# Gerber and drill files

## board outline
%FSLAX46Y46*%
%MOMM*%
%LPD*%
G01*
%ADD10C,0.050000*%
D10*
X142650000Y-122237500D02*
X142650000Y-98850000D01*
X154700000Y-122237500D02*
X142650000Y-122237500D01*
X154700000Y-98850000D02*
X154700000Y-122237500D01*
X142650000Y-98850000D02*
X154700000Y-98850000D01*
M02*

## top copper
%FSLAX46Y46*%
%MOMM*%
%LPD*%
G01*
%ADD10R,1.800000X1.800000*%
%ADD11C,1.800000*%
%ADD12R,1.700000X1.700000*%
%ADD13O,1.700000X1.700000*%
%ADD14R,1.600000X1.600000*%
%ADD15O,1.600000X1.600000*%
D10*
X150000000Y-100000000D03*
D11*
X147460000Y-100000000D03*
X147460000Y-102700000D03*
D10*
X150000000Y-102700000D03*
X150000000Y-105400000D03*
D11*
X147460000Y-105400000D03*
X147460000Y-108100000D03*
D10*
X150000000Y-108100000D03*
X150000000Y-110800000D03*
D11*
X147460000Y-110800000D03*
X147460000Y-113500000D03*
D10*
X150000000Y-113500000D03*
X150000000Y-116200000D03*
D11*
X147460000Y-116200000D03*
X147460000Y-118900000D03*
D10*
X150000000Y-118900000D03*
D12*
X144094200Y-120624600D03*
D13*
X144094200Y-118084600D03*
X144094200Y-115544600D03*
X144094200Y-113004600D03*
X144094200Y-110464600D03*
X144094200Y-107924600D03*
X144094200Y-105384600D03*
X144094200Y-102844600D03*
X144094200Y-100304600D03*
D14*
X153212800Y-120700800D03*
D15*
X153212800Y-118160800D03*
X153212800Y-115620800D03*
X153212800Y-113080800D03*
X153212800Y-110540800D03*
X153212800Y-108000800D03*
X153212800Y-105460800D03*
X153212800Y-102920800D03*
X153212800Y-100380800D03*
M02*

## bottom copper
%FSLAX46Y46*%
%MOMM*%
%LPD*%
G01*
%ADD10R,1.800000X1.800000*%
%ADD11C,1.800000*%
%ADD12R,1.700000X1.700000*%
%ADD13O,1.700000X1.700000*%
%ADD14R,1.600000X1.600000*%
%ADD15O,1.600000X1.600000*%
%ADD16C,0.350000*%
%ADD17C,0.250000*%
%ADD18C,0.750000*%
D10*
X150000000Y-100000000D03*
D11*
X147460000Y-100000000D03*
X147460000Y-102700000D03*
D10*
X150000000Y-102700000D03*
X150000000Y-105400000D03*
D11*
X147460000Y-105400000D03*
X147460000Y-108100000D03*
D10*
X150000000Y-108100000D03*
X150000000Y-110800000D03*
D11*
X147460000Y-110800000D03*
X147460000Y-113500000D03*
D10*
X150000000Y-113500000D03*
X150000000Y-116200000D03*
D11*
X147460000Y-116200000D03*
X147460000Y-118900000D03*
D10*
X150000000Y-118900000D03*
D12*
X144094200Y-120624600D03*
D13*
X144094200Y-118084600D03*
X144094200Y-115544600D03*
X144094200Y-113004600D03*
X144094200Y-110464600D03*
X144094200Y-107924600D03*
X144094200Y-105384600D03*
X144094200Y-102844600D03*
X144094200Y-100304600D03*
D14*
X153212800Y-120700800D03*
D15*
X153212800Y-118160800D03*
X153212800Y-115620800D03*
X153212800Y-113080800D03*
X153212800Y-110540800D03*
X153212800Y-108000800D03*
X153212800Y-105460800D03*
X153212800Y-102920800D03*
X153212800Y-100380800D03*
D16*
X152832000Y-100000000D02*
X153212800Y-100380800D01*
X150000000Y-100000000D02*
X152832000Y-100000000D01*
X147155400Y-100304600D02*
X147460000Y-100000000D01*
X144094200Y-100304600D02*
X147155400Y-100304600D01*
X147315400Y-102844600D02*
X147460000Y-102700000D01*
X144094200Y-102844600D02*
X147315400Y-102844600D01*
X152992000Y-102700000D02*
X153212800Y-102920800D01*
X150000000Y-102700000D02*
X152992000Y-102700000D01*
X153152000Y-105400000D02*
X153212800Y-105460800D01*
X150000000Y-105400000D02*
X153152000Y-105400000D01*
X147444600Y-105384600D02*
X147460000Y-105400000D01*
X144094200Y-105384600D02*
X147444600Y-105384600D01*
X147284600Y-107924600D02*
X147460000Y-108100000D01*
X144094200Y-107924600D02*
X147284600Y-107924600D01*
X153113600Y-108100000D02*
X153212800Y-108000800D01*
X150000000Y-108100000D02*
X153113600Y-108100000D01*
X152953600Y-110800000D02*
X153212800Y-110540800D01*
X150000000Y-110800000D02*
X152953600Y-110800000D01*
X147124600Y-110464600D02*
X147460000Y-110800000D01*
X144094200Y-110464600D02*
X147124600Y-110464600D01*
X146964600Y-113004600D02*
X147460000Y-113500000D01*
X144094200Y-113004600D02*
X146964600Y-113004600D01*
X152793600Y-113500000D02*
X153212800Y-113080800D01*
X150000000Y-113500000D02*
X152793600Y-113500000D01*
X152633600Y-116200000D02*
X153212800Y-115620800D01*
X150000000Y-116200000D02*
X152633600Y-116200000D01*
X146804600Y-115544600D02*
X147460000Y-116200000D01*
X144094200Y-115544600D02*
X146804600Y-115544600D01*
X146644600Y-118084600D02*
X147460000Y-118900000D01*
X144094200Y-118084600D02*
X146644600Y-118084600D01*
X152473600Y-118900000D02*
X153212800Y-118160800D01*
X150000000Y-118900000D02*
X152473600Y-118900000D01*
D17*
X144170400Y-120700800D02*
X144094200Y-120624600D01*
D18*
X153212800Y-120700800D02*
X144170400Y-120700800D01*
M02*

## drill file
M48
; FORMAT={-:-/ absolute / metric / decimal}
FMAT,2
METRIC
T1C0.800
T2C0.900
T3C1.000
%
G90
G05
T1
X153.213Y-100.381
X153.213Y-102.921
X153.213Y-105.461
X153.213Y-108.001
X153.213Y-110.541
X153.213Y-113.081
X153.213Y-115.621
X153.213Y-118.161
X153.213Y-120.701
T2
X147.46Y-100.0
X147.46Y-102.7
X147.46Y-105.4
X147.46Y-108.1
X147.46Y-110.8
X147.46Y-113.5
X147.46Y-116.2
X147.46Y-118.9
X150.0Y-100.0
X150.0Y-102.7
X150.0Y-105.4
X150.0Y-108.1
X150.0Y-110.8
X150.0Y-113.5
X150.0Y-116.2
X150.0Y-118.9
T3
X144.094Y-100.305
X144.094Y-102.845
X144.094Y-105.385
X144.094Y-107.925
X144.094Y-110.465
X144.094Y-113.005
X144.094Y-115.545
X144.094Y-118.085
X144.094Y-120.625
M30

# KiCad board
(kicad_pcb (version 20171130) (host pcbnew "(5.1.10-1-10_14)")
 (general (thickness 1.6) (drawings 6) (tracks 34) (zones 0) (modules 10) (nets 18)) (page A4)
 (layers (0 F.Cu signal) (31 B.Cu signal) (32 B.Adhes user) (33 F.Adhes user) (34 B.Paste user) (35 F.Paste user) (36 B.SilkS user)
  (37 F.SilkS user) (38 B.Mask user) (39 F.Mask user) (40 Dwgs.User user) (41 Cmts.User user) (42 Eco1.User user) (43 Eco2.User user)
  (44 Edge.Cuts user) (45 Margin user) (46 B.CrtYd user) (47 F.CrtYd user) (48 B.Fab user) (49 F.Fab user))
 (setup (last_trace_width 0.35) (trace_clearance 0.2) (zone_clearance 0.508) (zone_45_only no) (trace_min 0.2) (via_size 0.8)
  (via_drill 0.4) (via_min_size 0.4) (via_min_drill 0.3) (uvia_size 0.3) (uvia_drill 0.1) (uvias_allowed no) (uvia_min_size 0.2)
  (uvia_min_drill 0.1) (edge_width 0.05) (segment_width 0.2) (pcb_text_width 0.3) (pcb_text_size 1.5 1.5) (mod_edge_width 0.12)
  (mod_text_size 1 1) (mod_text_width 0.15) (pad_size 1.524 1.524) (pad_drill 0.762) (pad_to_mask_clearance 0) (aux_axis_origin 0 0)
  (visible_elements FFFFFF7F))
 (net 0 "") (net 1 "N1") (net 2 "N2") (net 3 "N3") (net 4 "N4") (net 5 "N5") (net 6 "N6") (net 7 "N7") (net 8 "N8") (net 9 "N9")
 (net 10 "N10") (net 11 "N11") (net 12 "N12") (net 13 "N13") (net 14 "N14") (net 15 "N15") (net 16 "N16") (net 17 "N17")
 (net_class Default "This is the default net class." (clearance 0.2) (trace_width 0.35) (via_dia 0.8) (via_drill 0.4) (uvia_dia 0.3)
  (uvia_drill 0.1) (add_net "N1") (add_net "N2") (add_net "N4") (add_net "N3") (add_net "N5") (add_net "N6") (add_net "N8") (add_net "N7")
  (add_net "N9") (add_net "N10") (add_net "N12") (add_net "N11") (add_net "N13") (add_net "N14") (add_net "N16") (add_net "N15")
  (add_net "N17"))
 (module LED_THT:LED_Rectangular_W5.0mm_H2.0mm (layer F.Cu) (at 150 100 180)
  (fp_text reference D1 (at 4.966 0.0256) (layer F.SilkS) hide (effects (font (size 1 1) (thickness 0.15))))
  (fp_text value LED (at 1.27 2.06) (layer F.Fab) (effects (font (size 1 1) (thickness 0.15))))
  (pad 1 thru_hole rect (at 0 0 180) (size 1.8 1.8) (drill 0.9) (layers *.Cu *.Mask) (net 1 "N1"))
  (pad 2 thru_hole circle (at 2.54 0 180) (size 1.8 1.8) (drill 0.9) (layers *.Cu *.Mask) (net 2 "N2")))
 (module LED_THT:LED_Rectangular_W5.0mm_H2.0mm (layer F.Cu) (at 150 102.7 180)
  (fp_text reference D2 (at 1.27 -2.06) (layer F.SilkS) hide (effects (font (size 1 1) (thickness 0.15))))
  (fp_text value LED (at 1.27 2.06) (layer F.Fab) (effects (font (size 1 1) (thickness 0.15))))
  (pad 2 thru_hole circle (at 2.54 0 180) (size 1.8 1.8) (drill 0.9) (layers *.Cu *.Mask) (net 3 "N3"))
  (pad 1 thru_hole rect (at 0 0 180) (size 1.8 1.8) (drill 0.9) (layers *.Cu *.Mask) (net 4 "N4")))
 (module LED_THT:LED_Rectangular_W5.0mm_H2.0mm (layer F.Cu) (at 150 105.4 180)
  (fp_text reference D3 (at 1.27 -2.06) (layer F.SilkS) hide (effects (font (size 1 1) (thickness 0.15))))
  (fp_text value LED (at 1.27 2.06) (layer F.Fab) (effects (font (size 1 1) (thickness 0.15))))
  (pad 1 thru_hole rect (at 0 0 180) (size 1.8 1.8) (drill 0.9) (layers *.Cu *.Mask) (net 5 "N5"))
  (pad 2 thru_hole circle (at 2.54 0 180) (size 1.8 1.8) (drill 0.9) (layers *.Cu *.Mask) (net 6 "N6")))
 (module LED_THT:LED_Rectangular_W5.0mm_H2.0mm (layer F.Cu) (at 150 108.1 180)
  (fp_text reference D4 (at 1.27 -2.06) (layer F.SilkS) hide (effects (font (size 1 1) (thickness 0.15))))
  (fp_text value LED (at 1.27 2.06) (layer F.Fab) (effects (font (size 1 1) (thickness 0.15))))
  (pad 2 thru_hole circle (at 2.54 0 180) (size 1.8 1.8) (drill 0.9) (layers *.Cu *.Mask) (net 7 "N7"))
  (pad 1 thru_hole rect (at 0 0 180) (size 1.8 1.8) (drill 0.9) (layers *.Cu *.Mask) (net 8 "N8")))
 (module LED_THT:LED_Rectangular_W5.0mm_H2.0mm (layer F.Cu) (at 150 110.8 180)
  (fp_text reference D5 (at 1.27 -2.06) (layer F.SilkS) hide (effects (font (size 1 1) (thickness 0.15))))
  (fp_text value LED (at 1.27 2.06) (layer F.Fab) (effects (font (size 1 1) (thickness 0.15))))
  (pad 1 thru_hole rect (at 0 0 180) (size 1.8 1.8) (drill 0.9) (layers *.Cu *.Mask) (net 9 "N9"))
  (pad 2 thru_hole circle (at 2.54 0 180) (size 1.8 1.8) (drill 0.9) (layers *.Cu *.Mask) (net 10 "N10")))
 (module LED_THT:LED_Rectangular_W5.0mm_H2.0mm (layer F.Cu) (at 150 113.5 180)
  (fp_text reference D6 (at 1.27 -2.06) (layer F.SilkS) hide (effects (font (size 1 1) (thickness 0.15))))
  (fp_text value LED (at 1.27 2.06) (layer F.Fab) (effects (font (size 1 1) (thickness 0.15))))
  (pad 2 thru_hole circle (at 2.54 0 180) (size 1.8 1.8) (drill 0.9) (layers *.Cu *.Mask) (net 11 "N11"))
  (pad 1 thru_hole rect (at 0 0 180) (size 1.8 1.8) (drill 0.9) (layers *.Cu *.Mask) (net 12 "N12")))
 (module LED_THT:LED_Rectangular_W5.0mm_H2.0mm (layer F.Cu) (at 150 116.2 180)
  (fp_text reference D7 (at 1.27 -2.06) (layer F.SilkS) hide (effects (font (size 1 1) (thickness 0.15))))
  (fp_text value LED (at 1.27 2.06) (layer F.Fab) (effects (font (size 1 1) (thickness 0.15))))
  (pad 1 thru_hole rect (at 0 0 180) (size 1.8 1.8) (drill 0.9) (layers *.Cu *.Mask) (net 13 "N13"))
  (pad 2 thru_hole circle (at 2.54 0 180) (size 1.8 1.8) (drill 0.9) (layers *.Cu *.Mask) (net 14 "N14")))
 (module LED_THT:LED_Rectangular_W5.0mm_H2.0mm (layer F.Cu) (at 150 118.9 180)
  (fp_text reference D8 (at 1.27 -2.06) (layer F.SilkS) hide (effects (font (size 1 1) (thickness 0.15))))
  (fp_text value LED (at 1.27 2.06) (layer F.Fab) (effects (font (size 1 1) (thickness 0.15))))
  (pad 2 thru_hole circle (at 2.54 0 180) (size 1.8 1.8) (drill 0.9) (layers *.Cu *.Mask) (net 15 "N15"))
  (pad 1 thru_hole rect (at 0 0 180) (size 1.8 1.8) (drill 0.9) (layers *.Cu *.Mask) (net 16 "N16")))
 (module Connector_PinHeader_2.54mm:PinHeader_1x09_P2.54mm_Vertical (layer F.Cu) (at 144.0942 120.6246 180)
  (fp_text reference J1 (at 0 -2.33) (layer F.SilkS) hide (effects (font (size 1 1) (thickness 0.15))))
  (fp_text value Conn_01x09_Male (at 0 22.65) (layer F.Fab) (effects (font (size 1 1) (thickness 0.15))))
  (pad 1 thru_hole rect (at 0 0 180) (size 1.7 1.7) (drill 1) (layers *.Cu *.Mask) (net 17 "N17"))
  (pad 2 thru_hole oval (at 0 2.54 180) (size 1.7 1.7) (drill 1) (layers *.Cu *.Mask) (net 15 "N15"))
  (pad 3 thru_hole oval (at 0 5.08 180) (size 1.7 1.7) (drill 1) (layers *.Cu *.Mask) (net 14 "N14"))
  (pad 4 thru_hole oval (at 0 7.62 180) (size 1.7 1.7) (drill 1) (layers *.Cu *.Mask) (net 11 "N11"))
  (pad 5 thru_hole oval (at 0 10.16 180) (size 1.7 1.7) (drill 1) (layers *.Cu *.Mask) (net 10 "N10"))
  (pad 6 thru_hole oval (at 0 12.7 180) (size 1.7 1.7) (drill 1) (layers *.Cu *.Mask) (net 7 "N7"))
  (pad 7 thru_hole oval (at 0 15.24 180) (size 1.7 1.7) (drill 1) (layers *.Cu *.Mask) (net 6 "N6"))
  (pad 8 thru_hole oval (at 0 17.78 180) (size 1.7 1.7) (drill 1) (layers *.Cu *.Mask) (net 3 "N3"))
  (pad 9 thru_hole oval (at 0 20.32 180) (size 1.7 1.7) (drill 1) (layers *.Cu *.Mask) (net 2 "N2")))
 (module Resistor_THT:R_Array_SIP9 (layer F.Cu) (at 153.2128 120.7008 90)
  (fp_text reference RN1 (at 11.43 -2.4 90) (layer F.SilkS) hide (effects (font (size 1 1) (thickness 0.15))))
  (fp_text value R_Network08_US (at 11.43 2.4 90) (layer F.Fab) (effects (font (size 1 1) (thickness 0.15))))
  (pad 1 thru_hole rect (at 0 0 90) (size 1.6 1.6) (drill 0.8) (layers *.Cu *.Mask) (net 17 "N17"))
  (pad 2 thru_hole oval (at 2.54 0 90) (size 1.6 1.6) (drill 0.8) (layers *.Cu *.Mask) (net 16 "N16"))
  (pad 3 thru_hole oval (at 5.08 0 90) (size 1.6 1.6) (drill 0.8) (layers *.Cu *.Mask) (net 13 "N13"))
  (pad 4 thru_hole oval (at 7.62 0 90) (size 1.6 1.6) (drill 0.8) (layers *.Cu *.Mask) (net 12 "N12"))
  (pad 5 thru_hole oval (at 10.16 0 90) (size 1.6 1.6) (drill 0.8) (layers *.Cu *.Mask) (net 9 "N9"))
  (pad 6 thru_hole oval (at 12.7 0 90) (size 1.6 1.6) (drill 0.8) (layers *.Cu *.Mask) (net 8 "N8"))
  (pad 7 thru_hole oval (at 15.24 0 90) (size 1.6 1.6) (drill 0.8) (layers *.Cu *.Mask) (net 5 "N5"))
  (pad 8 thru_hole oval (at 17.78 0 90) (size 1.6 1.6) (drill 0.8) (layers *.Cu *.Mask) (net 4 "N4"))
  (pad 9 thru_hole oval (at 20.32 0 90) (size 1.6 1.6) (drill 0.8) (layers *.Cu *.Mask) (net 1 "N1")))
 (gr_line (start 142.65 122.2375) (end 142.65 98.85) (layer Edge.Cuts) (width 0.05))
 (gr_line (start 154.7 122.2375) (end 142.65 122.2375) (layer Edge.Cuts) (width 0.05))
 (gr_line (start 154.7 98.85) (end 154.7 122.2375) (layer Edge.Cuts) (width 0.05))
 (gr_line (start 142.65 98.85) (end 154.7 98.85) (layer Edge.Cuts) (width 0.05))
 (segment (start 152.832 100) (end 153.2128 100.3808) (width 0.35) (layer B.Cu) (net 1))
 (segment (start 150 100) (end 152.832 100) (width 0.35) (layer B.Cu) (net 1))
 (segment (start 147.1554 100.3046) (end 147.46 100) (width 0.35) (layer B.Cu) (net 2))
 (segment (start 144.0942 100.3046) (end 147.1554 100.3046) (width 0.35) (layer B.Cu) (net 2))
 (segment (start 147.3154 102.8446) (end 147.46 102.7) (width 0.35) (layer B.Cu) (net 3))
 (segment (start 144.0942 102.8446) (end 147.3154 102.8446) (width 0.35) (layer B.Cu) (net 3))
 (segment (start 152.992 102.7) (end 153.2128 102.9208) (width 0.35) (layer B.Cu) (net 4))
 (segment (start 150 102.7) (end 152.992 102.7) (width 0.35) (layer B.Cu) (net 4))
 (segment (start 153.152 105.4) (end 153.2128 105.4608) (width 0.35) (layer B.Cu) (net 5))
 (segment (start 150 105.4) (end 153.152 105.4) (width 0.35) (layer B.Cu) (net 5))
 (segment (start 147.4446 105.3846) (end 147.46 105.4) (width 0.35) (layer B.Cu) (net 6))
 (segment (start 144.0942 105.3846) (end 147.4446 105.3846) (width 0.35) (layer B.Cu) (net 6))
 (segment (start 147.2846 107.9246) (end 147.46 108.1) (width 0.35) (layer B.Cu) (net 7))
 (segment (start 144.0942 107.9246) (end 147.2846 107.9246) (width 0.35) (layer B.Cu) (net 7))
 (segment (start 153.1136 108.1) (end 153.2128 108.0008) (width 0.35) (layer B.Cu) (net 8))
 (segment (start 150 108.1) (end 153.1136 108.1) (width 0.35) (layer B.Cu) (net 8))
 (segment (start 152.9536 110.8) (end 153.2128 110.5408) (width 0.35) (layer B.Cu) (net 9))
 (segment (start 150 110.8) (end 152.9536 110.8) (width 0.35) (layer B.Cu) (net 9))
 (segment (start 147.1246 110.4646) (end 147.46 110.8) (width 0.35) (layer B.Cu) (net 10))
 (segment (start 144.0942 110.4646) (end 147.1246 110.4646) (width 0.35) (layer B.Cu) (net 10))
 (segment (start 146.9646 113.0046) (end 147.46 113.5) (width 0.35) (layer B.Cu) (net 11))
 (segment (start 144.0942 113.0046) (end 146.9646 113.0046) (width 0.35) (layer B.Cu) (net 11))
 (segment (start 152.7936 113.5) (end 153.2128 113.0808) (width 0.35) (layer B.Cu) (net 12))
 (segment (start 150 113.5) (end 152.7936 113.5) (width 0.35) (layer B.Cu) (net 12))
 (segment (start 152.6336 116.2) (end 153.2128 115.6208) (width 0.35) (layer B.Cu) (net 13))
 (segment (start 150 116.2) (end 152.6336 116.2) (width 0.35) (layer B.Cu) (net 13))
 (segment (start 146.8046 115.5446) (end 147.46 116.2) (width 0.35) (layer B.Cu) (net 14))
 (segment (start 144.0942 115.5446) (end 146.8046 115.5446) (width 0.35) (layer B.Cu) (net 14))
 (segment (start 146.6446 118.0846) (end 147.46 118.9) (width 0.35) (layer B.Cu) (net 15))
 (segment (start 144.0942 118.0846) (end 146.6446 118.0846) (width 0.35) (layer B.Cu) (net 15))
 (segment (start 152.4736 118.9) (end 153.2128 118.1608) (width 0.35) (layer B.Cu) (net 16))
 (segment (start 150 118.9) (end 152.4736 118.9) (width 0.35) (layer B.Cu) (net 16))
 (segment (start 144.1704 120.7008) (end 144.0942 120.6246) (width 0.25) (layer B.Cu) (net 17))
 (segment (start 153.2128 120.7008) (end 144.1704 120.7008) (width 0.75) (layer B.Cu) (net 17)))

